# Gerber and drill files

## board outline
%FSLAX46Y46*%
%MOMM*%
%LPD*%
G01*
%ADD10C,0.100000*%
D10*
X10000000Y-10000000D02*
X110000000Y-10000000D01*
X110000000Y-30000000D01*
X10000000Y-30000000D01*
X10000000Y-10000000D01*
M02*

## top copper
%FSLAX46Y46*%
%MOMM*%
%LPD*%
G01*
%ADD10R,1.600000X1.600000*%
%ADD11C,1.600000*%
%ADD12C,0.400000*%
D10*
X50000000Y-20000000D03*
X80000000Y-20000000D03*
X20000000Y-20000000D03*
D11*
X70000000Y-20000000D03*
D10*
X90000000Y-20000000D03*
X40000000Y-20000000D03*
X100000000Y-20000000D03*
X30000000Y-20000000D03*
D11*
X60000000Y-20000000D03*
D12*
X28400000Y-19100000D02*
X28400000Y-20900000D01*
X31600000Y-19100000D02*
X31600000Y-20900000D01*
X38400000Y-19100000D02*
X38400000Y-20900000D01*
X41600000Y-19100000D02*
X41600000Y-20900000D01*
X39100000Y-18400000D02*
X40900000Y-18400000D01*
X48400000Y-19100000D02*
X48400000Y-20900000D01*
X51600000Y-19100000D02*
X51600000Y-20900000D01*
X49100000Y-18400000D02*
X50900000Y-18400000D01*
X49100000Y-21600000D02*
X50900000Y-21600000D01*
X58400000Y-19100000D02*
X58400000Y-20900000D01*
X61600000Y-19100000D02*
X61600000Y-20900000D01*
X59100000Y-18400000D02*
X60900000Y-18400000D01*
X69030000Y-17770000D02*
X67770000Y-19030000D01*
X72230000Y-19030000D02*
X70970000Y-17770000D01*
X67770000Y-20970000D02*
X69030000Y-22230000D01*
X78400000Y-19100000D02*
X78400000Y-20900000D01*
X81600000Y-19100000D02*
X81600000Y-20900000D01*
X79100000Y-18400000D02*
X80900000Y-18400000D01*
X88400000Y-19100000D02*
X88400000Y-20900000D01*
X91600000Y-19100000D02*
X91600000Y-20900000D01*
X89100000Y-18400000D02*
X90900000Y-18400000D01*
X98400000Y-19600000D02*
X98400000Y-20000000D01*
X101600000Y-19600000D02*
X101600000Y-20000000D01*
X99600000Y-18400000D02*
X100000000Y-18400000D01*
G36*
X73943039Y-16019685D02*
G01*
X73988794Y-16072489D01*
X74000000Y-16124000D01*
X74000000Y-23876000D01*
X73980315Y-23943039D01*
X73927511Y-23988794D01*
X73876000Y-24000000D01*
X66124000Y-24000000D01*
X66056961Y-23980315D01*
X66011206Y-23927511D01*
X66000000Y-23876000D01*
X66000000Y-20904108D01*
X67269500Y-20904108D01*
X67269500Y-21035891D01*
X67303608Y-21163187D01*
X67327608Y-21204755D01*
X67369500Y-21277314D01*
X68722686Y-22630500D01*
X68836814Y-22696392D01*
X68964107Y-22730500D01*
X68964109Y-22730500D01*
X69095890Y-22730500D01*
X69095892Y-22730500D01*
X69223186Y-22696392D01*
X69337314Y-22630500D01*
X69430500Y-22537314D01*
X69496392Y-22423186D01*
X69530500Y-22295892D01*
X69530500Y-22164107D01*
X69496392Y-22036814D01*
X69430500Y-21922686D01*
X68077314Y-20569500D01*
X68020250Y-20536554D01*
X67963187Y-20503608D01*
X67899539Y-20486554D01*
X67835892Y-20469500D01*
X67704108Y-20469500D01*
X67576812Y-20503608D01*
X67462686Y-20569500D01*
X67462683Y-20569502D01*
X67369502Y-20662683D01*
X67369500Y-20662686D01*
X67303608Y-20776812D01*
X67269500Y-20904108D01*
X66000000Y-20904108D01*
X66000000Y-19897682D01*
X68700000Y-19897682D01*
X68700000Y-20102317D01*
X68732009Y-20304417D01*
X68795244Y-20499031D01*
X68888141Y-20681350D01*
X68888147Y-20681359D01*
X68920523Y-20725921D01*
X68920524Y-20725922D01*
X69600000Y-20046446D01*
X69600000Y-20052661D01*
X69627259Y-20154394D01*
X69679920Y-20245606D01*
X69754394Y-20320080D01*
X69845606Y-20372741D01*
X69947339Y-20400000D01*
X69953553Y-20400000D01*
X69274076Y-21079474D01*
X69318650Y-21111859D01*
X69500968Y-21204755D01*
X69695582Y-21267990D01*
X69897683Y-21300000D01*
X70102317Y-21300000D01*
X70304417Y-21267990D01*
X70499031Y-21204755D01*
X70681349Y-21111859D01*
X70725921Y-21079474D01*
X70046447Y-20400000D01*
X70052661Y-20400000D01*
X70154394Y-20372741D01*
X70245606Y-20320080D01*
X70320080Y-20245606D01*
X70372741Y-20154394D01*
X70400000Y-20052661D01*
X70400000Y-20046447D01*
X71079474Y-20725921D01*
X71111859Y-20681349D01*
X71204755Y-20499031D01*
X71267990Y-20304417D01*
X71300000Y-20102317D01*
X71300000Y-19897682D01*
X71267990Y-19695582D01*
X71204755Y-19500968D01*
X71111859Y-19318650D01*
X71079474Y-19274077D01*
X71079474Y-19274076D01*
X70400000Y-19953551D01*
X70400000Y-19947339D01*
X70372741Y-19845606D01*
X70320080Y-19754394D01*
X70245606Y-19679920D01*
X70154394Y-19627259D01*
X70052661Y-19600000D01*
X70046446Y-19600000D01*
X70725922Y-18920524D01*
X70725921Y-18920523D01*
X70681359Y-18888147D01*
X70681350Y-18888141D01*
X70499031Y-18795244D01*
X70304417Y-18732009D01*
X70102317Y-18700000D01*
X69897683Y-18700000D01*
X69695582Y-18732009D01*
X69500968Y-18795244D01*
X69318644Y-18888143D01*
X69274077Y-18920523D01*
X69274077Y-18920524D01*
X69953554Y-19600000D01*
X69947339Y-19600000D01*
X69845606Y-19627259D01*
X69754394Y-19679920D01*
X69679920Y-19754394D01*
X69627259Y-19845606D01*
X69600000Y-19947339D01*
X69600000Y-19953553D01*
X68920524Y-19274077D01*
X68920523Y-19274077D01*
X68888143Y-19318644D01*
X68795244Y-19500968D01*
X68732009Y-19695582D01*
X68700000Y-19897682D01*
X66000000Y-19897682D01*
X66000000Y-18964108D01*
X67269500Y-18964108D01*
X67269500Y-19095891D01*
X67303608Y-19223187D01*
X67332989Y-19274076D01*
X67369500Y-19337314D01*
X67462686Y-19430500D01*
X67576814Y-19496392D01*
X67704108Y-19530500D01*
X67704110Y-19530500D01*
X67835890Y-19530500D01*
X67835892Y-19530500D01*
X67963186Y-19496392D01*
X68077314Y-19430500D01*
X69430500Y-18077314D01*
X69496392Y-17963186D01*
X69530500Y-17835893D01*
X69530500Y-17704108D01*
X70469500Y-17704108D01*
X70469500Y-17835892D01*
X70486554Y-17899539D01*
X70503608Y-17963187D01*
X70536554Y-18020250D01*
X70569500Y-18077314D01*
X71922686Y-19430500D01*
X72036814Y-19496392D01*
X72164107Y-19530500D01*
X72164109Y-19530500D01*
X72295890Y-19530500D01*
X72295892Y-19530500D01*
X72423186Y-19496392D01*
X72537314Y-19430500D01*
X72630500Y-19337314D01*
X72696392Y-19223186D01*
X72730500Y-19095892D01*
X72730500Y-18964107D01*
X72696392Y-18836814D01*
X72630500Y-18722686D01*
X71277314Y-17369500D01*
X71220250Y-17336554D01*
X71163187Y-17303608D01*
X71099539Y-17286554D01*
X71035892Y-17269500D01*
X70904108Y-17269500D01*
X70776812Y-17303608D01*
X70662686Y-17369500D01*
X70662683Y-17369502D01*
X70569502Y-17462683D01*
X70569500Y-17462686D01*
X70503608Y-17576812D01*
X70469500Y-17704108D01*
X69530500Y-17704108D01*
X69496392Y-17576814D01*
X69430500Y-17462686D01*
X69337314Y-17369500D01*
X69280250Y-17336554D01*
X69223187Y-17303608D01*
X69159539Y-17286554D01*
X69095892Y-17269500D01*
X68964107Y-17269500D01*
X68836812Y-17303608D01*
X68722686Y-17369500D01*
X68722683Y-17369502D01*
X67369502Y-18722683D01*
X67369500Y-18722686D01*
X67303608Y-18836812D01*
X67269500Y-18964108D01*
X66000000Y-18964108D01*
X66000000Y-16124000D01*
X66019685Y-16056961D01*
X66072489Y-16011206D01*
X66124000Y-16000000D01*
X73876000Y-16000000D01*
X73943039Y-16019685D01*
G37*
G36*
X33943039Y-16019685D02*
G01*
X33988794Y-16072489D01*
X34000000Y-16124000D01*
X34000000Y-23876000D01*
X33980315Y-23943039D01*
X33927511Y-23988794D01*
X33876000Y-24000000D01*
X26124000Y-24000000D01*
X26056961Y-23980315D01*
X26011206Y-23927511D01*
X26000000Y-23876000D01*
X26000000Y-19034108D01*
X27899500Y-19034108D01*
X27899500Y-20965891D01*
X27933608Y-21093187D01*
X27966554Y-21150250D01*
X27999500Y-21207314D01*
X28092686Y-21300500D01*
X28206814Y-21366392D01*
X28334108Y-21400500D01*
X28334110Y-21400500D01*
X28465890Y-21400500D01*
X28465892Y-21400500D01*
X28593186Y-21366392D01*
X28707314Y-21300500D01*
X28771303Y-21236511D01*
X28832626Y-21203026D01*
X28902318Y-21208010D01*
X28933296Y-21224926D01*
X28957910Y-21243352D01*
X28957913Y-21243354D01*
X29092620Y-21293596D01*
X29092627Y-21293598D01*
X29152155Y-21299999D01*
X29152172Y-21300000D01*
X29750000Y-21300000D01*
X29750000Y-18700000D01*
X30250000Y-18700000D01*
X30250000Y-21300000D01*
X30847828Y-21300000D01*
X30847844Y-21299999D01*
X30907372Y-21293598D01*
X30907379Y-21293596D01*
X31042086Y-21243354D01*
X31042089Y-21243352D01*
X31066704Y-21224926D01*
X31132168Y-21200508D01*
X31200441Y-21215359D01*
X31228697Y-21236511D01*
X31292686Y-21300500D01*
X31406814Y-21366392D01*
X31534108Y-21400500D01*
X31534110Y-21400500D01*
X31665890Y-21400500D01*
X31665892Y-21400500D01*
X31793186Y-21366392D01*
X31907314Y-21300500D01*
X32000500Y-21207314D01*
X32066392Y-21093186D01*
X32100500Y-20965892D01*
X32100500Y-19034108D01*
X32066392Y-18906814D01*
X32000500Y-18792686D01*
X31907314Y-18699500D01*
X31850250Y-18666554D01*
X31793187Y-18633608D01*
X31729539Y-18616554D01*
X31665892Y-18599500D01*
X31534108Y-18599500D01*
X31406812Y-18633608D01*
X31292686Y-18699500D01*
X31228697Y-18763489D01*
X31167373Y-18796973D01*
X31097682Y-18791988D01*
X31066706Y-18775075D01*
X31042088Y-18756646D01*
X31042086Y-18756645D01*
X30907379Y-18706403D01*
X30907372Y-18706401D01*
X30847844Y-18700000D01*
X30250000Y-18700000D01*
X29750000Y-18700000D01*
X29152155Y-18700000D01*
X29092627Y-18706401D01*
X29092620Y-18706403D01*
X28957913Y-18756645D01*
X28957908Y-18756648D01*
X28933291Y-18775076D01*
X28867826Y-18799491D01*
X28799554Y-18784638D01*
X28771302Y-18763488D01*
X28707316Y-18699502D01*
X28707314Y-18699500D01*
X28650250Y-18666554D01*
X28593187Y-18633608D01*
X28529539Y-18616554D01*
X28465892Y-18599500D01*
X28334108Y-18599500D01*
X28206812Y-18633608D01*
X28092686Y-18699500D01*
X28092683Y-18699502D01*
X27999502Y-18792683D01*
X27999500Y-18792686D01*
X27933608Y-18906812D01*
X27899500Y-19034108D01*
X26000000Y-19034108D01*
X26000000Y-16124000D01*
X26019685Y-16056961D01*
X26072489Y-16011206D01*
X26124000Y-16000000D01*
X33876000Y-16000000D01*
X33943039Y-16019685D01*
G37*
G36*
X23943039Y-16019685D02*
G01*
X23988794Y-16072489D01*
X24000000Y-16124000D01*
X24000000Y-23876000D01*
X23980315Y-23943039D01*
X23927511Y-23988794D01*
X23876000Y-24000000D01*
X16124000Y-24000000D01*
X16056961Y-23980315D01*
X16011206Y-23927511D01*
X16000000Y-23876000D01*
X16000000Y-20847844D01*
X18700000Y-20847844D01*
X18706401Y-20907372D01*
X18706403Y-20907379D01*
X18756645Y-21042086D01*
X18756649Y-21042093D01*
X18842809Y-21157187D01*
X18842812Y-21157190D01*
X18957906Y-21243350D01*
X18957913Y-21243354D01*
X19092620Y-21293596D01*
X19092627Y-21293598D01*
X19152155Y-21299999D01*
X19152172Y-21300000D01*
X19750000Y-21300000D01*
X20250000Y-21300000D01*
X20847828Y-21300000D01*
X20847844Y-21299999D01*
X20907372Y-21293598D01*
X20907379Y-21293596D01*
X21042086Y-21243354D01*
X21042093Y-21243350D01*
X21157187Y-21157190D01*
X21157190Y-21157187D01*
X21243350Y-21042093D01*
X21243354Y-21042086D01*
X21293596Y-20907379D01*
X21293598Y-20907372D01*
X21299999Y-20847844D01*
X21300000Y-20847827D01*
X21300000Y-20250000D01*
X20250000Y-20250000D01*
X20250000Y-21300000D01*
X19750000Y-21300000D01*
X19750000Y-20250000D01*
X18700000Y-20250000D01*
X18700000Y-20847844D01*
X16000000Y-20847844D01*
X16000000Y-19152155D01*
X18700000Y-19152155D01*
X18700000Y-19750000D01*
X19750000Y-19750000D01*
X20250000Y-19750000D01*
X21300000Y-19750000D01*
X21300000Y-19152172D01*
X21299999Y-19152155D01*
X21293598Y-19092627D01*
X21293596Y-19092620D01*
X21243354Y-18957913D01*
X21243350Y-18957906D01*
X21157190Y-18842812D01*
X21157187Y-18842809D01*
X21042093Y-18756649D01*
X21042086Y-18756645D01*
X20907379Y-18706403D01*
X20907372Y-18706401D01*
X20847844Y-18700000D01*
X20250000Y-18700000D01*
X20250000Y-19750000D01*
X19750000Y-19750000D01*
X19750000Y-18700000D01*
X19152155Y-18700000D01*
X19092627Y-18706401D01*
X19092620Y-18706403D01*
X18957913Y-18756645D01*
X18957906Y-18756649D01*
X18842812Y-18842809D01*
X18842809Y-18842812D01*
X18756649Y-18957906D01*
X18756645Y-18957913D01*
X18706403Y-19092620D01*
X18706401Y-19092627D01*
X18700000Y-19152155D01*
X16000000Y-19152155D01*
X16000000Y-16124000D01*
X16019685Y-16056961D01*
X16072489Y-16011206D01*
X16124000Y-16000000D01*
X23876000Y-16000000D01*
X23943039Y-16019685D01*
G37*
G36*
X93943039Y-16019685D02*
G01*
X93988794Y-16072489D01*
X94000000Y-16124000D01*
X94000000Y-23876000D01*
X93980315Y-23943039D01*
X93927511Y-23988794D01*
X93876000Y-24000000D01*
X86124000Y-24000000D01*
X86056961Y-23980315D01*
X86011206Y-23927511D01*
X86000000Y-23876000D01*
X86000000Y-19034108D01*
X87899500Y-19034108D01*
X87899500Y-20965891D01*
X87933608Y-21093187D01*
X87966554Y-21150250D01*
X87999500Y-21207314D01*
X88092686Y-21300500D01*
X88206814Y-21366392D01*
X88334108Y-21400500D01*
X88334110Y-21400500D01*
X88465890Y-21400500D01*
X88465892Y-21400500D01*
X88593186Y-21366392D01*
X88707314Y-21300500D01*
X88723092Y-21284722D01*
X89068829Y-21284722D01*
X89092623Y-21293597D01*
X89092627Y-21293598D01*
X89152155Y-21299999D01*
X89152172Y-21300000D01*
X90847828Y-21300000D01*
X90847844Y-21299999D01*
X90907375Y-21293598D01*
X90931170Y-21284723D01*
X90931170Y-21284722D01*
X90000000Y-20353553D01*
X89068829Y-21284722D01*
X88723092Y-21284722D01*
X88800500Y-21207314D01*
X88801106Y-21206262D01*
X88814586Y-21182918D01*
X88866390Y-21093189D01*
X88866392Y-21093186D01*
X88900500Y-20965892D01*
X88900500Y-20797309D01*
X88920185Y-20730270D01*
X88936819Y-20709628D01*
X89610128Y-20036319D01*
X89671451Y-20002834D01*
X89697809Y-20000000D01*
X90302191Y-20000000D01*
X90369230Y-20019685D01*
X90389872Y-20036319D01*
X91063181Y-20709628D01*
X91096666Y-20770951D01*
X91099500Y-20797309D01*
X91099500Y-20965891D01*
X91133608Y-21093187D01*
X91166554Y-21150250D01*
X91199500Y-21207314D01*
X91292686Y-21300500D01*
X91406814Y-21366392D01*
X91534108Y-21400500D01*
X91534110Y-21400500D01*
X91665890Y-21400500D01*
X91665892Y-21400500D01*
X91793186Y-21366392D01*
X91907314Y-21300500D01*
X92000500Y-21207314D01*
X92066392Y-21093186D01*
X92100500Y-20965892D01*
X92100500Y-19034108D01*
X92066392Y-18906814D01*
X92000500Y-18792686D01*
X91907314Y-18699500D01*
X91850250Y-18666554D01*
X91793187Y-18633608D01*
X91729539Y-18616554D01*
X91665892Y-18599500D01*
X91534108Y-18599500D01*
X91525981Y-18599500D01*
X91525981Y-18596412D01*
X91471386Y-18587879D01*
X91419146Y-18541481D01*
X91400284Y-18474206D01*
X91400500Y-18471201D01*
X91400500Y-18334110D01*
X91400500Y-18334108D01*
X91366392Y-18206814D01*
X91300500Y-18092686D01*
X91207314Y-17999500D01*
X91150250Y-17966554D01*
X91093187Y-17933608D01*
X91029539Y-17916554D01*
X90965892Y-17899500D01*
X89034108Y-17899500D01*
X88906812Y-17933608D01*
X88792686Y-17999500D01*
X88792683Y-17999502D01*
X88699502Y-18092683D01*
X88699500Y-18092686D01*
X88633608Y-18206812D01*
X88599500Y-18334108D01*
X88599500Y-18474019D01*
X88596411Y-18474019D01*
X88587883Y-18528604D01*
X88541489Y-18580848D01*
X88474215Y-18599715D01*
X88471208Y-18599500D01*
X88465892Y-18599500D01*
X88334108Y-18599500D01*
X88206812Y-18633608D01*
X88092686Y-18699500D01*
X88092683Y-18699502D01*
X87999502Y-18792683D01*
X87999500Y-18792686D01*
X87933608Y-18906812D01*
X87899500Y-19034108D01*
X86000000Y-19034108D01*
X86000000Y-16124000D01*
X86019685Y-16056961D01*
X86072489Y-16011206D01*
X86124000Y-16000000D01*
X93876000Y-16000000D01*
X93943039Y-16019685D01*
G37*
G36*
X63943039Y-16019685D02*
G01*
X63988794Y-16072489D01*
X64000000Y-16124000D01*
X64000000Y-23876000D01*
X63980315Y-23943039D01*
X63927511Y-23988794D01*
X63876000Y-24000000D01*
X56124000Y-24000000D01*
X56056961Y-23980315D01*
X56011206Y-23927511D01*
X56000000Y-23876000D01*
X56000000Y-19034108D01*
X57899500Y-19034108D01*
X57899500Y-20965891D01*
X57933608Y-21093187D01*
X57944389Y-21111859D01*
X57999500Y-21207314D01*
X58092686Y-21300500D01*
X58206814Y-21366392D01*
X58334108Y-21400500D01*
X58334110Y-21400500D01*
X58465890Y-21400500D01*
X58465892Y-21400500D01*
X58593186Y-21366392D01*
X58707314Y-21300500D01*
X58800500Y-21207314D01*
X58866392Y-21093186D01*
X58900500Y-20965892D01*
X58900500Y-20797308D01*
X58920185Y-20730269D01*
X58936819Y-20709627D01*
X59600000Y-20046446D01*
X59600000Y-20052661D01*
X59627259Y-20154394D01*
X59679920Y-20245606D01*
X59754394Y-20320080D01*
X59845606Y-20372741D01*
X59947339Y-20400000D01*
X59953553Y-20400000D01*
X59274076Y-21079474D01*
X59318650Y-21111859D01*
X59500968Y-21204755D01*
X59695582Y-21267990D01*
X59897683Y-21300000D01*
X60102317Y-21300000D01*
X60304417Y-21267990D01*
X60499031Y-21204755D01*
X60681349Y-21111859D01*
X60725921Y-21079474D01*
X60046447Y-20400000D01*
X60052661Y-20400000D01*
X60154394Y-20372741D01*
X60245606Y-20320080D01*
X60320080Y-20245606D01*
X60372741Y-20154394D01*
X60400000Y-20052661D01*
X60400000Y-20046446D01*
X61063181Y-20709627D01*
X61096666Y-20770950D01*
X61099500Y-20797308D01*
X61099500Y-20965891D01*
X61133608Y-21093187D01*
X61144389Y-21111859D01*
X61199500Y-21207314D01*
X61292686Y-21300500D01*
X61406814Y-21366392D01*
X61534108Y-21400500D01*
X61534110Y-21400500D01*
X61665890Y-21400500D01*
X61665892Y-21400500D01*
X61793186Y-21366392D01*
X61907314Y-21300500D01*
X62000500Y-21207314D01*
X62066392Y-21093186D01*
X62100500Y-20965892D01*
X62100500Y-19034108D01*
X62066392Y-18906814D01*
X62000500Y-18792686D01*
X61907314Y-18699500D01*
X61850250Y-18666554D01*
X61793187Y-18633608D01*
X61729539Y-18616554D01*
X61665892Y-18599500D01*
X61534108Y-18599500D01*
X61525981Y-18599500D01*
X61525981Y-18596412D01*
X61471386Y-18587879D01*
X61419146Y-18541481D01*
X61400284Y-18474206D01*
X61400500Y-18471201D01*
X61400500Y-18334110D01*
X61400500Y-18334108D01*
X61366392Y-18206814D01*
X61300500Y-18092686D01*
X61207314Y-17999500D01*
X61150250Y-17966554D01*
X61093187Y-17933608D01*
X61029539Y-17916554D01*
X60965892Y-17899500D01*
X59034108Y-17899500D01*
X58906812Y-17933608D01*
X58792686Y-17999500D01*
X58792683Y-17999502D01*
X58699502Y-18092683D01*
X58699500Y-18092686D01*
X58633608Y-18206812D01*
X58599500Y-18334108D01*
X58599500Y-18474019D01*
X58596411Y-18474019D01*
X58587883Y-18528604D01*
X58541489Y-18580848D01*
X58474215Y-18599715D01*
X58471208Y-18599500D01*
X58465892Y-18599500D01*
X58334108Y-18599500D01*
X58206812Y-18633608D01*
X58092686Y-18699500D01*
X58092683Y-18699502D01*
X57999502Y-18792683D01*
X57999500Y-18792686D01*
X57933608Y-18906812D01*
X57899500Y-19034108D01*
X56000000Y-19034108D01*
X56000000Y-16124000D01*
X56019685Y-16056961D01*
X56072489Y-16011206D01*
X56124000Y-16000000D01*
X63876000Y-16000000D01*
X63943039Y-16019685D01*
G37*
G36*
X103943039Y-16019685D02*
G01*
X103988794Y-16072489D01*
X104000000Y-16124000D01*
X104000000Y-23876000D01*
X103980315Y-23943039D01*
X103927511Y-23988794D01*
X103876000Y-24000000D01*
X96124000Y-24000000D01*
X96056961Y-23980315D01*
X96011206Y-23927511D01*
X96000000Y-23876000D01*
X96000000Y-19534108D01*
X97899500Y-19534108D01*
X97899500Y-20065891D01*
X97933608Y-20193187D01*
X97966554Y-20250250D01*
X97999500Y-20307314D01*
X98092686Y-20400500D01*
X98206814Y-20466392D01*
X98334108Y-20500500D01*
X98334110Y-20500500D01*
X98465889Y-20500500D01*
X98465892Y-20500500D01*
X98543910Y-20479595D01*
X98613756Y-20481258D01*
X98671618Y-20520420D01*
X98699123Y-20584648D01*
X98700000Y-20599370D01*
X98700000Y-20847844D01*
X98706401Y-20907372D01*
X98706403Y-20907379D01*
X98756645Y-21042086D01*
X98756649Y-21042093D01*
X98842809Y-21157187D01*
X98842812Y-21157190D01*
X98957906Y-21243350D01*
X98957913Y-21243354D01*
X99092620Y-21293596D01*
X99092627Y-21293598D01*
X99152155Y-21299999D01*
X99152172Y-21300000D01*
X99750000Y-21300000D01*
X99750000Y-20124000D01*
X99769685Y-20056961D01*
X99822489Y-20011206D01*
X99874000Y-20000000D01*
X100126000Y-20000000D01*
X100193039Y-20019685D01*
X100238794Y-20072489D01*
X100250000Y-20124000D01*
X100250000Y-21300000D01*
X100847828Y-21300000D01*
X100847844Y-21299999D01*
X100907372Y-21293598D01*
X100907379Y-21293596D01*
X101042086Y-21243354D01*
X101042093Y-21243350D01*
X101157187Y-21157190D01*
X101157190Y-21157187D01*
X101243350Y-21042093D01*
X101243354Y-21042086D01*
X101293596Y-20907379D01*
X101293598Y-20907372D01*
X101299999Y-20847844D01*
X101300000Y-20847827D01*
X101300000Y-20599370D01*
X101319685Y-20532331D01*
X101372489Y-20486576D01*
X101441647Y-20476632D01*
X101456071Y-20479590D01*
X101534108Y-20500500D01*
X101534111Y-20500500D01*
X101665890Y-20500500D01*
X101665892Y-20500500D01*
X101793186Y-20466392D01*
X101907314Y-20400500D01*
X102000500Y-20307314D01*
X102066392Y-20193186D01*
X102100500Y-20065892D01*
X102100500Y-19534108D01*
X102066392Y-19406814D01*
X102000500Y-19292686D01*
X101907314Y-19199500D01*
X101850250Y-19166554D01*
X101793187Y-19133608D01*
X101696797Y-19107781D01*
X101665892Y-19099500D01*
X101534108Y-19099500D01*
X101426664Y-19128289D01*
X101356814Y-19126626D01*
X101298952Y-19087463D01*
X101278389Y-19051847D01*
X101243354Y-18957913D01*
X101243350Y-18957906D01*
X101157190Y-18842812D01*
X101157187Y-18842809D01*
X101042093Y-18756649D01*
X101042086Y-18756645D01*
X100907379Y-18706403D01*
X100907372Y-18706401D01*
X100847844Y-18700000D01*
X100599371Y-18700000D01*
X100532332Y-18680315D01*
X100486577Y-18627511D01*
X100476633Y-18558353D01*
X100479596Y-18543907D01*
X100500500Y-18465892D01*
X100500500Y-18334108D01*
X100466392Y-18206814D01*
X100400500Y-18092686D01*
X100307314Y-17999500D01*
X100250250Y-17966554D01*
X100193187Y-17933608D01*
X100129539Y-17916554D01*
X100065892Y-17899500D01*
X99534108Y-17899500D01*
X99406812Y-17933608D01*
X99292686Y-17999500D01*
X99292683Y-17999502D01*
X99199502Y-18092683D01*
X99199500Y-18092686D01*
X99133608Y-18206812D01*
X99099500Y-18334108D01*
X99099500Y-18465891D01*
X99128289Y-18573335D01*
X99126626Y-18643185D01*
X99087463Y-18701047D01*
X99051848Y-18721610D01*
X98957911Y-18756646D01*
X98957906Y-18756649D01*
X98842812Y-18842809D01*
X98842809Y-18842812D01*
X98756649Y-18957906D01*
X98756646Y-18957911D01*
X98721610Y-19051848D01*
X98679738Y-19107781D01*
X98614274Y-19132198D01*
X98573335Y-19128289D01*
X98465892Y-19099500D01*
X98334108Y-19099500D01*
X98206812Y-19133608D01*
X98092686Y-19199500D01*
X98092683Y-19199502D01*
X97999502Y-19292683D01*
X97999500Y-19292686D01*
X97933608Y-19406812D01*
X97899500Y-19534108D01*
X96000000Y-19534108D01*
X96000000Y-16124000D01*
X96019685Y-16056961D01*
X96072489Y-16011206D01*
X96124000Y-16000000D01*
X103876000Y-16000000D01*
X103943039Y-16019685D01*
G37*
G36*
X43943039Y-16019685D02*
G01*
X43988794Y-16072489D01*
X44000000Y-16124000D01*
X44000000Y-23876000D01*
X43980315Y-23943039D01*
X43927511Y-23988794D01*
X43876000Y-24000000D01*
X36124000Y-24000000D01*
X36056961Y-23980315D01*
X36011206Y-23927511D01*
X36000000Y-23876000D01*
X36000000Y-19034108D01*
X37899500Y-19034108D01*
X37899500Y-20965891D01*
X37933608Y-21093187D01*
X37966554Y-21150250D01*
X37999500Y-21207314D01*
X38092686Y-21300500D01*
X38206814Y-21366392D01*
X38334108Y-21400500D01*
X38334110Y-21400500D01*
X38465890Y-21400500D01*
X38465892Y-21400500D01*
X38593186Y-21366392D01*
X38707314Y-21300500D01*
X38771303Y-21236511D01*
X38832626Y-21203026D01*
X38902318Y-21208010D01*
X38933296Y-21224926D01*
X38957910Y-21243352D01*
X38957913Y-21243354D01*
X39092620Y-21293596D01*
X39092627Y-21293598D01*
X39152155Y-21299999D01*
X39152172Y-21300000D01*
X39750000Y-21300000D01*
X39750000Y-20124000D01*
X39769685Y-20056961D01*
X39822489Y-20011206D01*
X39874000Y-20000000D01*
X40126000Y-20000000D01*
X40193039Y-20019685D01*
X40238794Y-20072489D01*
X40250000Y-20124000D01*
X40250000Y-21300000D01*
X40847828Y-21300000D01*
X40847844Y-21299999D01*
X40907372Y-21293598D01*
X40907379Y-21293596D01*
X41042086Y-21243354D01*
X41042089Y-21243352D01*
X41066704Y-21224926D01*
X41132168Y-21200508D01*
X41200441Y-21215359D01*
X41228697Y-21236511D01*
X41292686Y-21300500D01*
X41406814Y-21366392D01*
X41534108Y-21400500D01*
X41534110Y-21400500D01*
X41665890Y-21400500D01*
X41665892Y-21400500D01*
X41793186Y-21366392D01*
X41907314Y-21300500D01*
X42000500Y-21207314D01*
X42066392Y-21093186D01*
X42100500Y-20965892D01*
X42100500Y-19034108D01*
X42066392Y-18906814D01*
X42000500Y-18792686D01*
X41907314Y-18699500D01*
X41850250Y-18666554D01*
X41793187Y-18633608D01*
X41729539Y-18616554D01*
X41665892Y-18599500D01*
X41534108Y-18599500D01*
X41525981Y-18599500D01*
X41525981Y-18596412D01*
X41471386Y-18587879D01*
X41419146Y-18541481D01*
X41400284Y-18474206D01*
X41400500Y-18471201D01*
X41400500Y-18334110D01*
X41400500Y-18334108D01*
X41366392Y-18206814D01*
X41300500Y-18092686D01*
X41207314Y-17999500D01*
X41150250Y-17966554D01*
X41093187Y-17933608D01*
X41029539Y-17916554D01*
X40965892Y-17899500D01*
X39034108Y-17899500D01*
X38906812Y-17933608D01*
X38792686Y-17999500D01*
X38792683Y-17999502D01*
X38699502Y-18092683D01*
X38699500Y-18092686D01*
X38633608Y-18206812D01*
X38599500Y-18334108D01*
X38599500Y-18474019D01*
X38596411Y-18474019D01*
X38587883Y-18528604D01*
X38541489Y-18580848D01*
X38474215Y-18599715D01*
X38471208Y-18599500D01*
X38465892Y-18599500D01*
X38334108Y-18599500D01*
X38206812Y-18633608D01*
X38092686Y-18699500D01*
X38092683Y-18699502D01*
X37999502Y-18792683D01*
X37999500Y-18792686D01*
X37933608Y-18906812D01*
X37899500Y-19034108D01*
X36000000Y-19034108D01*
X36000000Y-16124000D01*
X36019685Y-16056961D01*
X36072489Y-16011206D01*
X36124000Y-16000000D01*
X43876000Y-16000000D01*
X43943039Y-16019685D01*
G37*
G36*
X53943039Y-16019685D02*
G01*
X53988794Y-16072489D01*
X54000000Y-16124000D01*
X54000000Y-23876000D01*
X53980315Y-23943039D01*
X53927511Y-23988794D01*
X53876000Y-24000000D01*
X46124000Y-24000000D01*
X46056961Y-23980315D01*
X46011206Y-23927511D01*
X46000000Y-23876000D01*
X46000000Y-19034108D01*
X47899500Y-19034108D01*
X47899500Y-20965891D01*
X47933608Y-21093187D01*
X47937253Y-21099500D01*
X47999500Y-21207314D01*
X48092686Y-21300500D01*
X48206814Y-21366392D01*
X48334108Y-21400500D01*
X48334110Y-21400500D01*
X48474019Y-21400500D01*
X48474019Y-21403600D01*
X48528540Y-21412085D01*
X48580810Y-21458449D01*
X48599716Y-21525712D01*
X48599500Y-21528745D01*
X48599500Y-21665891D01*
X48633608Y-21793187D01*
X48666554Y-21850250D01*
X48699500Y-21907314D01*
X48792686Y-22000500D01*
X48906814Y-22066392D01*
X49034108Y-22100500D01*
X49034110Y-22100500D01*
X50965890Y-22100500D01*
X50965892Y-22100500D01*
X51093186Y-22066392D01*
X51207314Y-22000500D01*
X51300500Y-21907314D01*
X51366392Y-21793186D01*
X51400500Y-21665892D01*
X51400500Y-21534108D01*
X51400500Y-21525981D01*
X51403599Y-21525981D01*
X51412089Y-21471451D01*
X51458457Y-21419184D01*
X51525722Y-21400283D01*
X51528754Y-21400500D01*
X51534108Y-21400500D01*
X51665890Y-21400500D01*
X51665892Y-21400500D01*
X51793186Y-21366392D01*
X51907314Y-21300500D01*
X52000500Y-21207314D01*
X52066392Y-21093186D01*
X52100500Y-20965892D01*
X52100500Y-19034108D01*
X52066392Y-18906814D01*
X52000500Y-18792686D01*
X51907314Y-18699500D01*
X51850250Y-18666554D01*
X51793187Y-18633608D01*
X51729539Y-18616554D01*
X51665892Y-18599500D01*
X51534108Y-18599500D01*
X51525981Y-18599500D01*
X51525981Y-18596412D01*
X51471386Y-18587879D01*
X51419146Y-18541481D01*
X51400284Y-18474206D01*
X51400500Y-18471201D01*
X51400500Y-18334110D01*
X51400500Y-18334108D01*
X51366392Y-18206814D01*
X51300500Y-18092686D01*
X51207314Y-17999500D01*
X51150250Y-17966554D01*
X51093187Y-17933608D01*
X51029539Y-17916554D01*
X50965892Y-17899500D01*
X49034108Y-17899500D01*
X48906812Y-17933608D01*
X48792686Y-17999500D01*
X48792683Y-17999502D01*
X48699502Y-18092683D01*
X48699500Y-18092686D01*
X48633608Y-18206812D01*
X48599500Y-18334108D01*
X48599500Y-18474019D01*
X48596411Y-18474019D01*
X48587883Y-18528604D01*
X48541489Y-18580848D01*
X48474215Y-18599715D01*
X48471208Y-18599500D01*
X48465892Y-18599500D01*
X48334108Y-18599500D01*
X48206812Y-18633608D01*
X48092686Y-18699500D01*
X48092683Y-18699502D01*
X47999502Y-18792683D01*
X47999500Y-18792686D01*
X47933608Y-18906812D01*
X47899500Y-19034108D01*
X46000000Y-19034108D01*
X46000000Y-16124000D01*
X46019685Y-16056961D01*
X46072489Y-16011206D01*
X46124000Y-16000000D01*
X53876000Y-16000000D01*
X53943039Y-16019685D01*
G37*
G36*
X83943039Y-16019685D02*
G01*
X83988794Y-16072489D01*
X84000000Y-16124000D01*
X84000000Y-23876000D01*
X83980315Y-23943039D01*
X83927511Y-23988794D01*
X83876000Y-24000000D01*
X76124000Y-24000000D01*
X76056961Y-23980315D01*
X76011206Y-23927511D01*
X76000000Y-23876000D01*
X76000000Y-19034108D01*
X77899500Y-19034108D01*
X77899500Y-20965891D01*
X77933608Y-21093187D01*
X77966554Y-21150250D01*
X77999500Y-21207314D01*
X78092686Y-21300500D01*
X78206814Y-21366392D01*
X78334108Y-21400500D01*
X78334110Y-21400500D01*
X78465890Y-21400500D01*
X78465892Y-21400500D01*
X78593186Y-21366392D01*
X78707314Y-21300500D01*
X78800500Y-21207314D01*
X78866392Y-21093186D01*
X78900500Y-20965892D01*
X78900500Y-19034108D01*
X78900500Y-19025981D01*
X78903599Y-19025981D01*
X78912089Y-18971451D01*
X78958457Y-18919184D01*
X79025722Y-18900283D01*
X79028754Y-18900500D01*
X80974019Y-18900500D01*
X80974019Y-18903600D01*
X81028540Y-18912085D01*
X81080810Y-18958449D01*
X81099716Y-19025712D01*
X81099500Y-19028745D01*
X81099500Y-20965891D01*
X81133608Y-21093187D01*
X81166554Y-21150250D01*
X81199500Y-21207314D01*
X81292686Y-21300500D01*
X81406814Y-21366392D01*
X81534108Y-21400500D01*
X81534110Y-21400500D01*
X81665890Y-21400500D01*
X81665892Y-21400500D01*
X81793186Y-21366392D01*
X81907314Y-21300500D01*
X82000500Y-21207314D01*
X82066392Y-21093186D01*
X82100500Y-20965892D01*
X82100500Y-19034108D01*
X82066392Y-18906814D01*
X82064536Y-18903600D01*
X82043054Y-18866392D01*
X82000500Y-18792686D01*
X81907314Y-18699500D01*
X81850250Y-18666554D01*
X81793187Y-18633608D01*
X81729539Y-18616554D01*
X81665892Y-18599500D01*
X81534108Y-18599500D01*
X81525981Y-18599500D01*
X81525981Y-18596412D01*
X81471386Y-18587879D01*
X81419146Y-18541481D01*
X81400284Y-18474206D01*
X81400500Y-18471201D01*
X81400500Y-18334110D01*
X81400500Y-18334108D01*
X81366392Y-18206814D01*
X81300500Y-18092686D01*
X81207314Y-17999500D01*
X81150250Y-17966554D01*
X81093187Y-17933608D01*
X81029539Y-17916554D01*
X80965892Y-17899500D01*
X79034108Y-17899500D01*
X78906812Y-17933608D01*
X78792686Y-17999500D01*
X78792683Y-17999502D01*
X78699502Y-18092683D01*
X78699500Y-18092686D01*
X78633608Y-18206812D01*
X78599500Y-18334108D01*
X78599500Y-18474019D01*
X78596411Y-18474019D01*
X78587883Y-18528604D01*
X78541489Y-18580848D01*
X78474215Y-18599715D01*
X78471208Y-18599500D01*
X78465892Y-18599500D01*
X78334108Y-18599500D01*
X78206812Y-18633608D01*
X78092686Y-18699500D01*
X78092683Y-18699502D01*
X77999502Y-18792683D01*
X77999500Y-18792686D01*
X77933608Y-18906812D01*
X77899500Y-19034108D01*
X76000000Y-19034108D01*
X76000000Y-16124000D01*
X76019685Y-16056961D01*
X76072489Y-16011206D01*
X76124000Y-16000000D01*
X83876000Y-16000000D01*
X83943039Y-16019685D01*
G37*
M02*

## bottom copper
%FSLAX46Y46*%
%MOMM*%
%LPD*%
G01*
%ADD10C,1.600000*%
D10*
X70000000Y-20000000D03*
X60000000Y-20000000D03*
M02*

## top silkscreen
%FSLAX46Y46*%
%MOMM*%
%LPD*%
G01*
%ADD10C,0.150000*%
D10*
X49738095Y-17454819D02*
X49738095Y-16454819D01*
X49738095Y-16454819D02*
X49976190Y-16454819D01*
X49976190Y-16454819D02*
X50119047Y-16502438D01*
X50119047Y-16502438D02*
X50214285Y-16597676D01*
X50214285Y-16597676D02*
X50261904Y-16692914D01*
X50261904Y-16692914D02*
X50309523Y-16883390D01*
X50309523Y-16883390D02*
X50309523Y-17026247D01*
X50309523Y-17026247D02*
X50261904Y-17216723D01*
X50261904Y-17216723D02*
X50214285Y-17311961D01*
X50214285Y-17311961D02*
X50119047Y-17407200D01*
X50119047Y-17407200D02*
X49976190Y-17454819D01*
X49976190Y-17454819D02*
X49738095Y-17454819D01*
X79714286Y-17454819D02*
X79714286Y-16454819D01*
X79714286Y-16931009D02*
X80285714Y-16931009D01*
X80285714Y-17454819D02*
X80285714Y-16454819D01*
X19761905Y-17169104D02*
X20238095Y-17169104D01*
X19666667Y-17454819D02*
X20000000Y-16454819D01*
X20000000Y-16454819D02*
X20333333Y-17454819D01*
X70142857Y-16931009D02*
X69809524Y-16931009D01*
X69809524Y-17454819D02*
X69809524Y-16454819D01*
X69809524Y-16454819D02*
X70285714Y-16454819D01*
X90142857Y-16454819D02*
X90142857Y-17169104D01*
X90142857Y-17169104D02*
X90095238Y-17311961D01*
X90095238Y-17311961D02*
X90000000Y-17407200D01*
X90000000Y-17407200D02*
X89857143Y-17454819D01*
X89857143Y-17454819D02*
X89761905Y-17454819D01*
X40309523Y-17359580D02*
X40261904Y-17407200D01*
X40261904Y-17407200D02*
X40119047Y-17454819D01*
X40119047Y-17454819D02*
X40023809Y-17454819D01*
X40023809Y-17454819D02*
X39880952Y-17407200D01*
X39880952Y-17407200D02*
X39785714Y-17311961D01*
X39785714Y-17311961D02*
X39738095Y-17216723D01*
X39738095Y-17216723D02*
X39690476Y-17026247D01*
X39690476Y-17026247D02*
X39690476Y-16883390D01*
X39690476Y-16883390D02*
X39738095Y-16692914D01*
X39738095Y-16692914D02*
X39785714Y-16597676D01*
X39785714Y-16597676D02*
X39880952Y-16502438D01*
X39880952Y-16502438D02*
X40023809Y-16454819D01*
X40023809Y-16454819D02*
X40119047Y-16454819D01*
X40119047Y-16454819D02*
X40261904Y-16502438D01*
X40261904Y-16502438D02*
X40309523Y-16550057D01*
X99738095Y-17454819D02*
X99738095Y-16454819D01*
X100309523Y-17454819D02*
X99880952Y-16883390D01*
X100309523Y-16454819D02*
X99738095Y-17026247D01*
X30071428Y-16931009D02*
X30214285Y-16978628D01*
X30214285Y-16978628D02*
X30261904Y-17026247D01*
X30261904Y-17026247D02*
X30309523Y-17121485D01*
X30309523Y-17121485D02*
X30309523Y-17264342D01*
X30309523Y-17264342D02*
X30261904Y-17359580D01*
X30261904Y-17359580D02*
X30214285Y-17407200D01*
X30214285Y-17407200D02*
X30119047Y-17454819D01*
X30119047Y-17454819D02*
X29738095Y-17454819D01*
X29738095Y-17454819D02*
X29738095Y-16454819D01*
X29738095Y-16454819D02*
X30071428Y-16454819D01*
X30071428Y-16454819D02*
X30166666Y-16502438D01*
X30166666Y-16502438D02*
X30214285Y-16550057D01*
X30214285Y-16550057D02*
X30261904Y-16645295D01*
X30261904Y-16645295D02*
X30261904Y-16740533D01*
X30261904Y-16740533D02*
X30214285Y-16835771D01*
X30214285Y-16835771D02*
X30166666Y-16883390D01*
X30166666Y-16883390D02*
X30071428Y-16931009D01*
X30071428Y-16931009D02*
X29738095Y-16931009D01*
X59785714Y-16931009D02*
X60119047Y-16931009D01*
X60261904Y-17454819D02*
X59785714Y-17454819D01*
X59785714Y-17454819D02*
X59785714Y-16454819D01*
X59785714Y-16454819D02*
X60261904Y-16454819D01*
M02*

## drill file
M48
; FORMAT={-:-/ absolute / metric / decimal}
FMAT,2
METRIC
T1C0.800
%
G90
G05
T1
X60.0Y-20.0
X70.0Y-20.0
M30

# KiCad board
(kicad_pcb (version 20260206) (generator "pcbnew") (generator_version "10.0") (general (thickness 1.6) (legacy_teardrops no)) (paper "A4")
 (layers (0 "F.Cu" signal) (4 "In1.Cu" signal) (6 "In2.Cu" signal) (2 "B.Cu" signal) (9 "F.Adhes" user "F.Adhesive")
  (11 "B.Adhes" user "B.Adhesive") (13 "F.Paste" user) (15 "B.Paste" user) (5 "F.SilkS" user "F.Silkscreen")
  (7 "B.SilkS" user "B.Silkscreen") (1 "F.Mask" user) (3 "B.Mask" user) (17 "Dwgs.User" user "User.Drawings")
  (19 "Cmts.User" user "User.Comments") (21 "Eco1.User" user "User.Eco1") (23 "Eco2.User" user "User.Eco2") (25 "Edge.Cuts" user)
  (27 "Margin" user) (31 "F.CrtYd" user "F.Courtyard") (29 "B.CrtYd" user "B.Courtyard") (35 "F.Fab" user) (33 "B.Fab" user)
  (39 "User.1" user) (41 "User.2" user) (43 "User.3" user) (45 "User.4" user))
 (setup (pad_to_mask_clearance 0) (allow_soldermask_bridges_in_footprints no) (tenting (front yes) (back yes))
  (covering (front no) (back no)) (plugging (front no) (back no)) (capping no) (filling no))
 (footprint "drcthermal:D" (layer "F.Cu") (at 50 20)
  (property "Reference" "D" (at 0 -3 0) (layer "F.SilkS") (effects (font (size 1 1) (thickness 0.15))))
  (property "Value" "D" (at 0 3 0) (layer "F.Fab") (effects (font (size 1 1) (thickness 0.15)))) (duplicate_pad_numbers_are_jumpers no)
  (pad "1" smd rect (at 0 0) (size 1.6 1.6) (layers "F.Cu" "F.Mask" "F.Paste") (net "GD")))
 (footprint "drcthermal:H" (layer "F.Cu") (at 80 20)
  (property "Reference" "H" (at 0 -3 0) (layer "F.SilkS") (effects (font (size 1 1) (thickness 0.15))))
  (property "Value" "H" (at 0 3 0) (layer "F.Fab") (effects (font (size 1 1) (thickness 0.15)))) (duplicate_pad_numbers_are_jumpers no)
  (pad "1" smd rect (at 0 0) (size 1.6 1.6) (layers "F.Cu" "F.Mask" "F.Paste") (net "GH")))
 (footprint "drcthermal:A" (layer "F.Cu") (at 20 20)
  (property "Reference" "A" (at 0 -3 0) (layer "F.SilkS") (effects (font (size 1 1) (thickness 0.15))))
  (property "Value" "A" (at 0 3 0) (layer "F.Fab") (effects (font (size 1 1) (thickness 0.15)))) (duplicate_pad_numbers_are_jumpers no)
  (pad "1" smd rect (at 0 0) (size 1.6 1.6) (layers "F.Cu" "F.Mask" "F.Paste") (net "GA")))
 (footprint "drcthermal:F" (layer "F.Cu") (at 70 20)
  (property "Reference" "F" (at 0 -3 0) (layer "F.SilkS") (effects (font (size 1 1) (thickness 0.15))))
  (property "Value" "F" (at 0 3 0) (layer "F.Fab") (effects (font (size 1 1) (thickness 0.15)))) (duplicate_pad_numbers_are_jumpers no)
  (pad "1" thru_hole circle (at 0 0) (size 1.6 1.6) (drill 0.8) (layers "*.Cu" "*.Mask") (remove_unused_layers no) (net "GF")))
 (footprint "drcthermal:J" (layer "F.Cu") (at 90 20)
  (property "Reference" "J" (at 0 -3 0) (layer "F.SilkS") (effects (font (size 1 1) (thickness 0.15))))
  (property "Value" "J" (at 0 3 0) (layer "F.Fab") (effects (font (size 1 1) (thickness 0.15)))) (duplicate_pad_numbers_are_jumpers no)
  (pad "1" smd rect (at 0 0) (size 1.6 1.6) (layers "F.Cu" "F.Mask" "F.Paste") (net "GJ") (thermal_bridge_angle 45)))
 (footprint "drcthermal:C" (layer "F.Cu") (at 40 20)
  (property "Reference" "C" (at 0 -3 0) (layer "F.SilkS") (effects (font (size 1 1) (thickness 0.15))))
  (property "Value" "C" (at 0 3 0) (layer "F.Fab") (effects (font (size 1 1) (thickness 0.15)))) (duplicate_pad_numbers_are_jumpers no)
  (pad "1" smd rect (at 0 0) (size 1.6 1.6) (layers "F.Cu" "F.Mask" "F.Paste") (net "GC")))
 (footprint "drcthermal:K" (layer "F.Cu") (at 100 20)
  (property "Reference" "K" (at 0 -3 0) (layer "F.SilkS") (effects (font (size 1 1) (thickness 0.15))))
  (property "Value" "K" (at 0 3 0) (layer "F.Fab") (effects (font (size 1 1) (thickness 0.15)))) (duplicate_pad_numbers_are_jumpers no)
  (pad "1" smd rect (at 0 0) (size 1.6 1.6) (layers "F.Cu" "F.Mask" "F.Paste") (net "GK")))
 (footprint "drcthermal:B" (layer "F.Cu") (at 30 20)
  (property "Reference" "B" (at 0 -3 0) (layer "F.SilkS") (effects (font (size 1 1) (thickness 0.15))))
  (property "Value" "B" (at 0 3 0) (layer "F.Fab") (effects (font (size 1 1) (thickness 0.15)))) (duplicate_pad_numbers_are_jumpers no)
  (pad "1" smd rect (at 0 0) (size 1.6 1.6) (layers "F.Cu" "F.Mask" "F.Paste") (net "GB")))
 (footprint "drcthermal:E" (layer "F.Cu") (at 60 20)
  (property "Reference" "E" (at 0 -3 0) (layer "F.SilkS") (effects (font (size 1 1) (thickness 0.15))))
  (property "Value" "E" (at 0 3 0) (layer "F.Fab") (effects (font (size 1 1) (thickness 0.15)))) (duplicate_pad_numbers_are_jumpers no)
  (pad "1" thru_hole circle (at 0 0) (size 1.6 1.6) (drill 0.8) (layers "*.Cu" "*.Mask") (remove_unused_layers no) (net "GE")))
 (gr_rect (start 10 10) (end 110 30) (stroke (width 0.1) (type solid)) (fill no) (layer "Edge.Cuts"))
 (segment (start 28.4 19.1) (end 28.4 20.9) (width 0.4) (layer "F.Cu") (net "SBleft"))
 (segment (start 31.6 19.1) (end 31.6 20.9) (width 0.4) (layer "F.Cu") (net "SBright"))
 (segment (start 38.4 19.1) (end 38.4 20.9) (width 0.4) (layer "F.Cu") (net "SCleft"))
 (segment (start 41.6 19.1) (end 41.6 20.9) (width 0.4) (layer "F.Cu") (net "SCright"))
 (segment (start 39.1 18.4) (end 40.9 18.4) (width 0.4) (layer "F.Cu") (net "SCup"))
 (segment (start 48.4 19.1) (end 48.4 20.9) (width 0.4) (layer "F.Cu") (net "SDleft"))
 (segment (start 51.6 19.1) (end 51.6 20.9) (width 0.4) (layer "F.Cu") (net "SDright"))
 (segment (start 49.1 18.4) (end 50.9 18.4) (width 0.4) (layer "F.Cu") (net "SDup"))
 (segment (start 49.1 21.6) (end 50.9 21.6) (width 0.4) (layer "F.Cu") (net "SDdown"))
 (segment (start 58.4 19.1) (end 58.4 20.9) (width 0.4) (layer "F.Cu") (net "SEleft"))
 (segment (start 61.6 19.1) (end 61.6 20.9) (width 0.4) (layer "F.Cu") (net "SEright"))
 (segment (start 59.1 18.4) (end 60.9 18.4) (width 0.4) (layer "F.Cu") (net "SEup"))
 (segment (start 69.03 17.77) (end 67.77 19.03) (width 0.4) (layer "F.Cu") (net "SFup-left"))
 (segment (start 72.23 19.03) (end 70.97 17.77) (width 0.4) (layer "F.Cu") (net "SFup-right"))
 (segment (start 67.77 20.97) (end 69.03 22.23) (width 0.4) (layer "F.Cu") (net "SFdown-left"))
 (segment (start 78.4 19.1) (end 78.4 20.9) (width 0.4) (layer "F.Cu") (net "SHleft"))
 (segment (start 81.6 19.1) (end 81.6 20.9) (width 0.4) (layer "F.Cu") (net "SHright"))
 (segment (start 79.1 18.4) (end 80.9 18.4) (width 0.4) (layer "F.Cu") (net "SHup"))
 (segment (start 88.4 19.1) (end 88.4 20.9) (width 0.4) (layer "F.Cu") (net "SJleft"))
 (segment (start 91.6 19.1) (end 91.6 20.9) (width 0.4) (layer "F.Cu") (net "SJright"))
 (segment (start 89.1 18.4) (end 90.9 18.4) (width 0.4) (layer "F.Cu") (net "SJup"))
 (segment (start 98.4 19.6) (end 98.4 20) (width 0.4) (layer "F.Cu") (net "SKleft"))
 (segment (start 101.6 19.6) (end 101.6 20) (width 0.4) (layer "F.Cu") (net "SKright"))
 (segment (start 99.6 18.4) (end 100 18.4) (width 0.4) (layer "F.Cu") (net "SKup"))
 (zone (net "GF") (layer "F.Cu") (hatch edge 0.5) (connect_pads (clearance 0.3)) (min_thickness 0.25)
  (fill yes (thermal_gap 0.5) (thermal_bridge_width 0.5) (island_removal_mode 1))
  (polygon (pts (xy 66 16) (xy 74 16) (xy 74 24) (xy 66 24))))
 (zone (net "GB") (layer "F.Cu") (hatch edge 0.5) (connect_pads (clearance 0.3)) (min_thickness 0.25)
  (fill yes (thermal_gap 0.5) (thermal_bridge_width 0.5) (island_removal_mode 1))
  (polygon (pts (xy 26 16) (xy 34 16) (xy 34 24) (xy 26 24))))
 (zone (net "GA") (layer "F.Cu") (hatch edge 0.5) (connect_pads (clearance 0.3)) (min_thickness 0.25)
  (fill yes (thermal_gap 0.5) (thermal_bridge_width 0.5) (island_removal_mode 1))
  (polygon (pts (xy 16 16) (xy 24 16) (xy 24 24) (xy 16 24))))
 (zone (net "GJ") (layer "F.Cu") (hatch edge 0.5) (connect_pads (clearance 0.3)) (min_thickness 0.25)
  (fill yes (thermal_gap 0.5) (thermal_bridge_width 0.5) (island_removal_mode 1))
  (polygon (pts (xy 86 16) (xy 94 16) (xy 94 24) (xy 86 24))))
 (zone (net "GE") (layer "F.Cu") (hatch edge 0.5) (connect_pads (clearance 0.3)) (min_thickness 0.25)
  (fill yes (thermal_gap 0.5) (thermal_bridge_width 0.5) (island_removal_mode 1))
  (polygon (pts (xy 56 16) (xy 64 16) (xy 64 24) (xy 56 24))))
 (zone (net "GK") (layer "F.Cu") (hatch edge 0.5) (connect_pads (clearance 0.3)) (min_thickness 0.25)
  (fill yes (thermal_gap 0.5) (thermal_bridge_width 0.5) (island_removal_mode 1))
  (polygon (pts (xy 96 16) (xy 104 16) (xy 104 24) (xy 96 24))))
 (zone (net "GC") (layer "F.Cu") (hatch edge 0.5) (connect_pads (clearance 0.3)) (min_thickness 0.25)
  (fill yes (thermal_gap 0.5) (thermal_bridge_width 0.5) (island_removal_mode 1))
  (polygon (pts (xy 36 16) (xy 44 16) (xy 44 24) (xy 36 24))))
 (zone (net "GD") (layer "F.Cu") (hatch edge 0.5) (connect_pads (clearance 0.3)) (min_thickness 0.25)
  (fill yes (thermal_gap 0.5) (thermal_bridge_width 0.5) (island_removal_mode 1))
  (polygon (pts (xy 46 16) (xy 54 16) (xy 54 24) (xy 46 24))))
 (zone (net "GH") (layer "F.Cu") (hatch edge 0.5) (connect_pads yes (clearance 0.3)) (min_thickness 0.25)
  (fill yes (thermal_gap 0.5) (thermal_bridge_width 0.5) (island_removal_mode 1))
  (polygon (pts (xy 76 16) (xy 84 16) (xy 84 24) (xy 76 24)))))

